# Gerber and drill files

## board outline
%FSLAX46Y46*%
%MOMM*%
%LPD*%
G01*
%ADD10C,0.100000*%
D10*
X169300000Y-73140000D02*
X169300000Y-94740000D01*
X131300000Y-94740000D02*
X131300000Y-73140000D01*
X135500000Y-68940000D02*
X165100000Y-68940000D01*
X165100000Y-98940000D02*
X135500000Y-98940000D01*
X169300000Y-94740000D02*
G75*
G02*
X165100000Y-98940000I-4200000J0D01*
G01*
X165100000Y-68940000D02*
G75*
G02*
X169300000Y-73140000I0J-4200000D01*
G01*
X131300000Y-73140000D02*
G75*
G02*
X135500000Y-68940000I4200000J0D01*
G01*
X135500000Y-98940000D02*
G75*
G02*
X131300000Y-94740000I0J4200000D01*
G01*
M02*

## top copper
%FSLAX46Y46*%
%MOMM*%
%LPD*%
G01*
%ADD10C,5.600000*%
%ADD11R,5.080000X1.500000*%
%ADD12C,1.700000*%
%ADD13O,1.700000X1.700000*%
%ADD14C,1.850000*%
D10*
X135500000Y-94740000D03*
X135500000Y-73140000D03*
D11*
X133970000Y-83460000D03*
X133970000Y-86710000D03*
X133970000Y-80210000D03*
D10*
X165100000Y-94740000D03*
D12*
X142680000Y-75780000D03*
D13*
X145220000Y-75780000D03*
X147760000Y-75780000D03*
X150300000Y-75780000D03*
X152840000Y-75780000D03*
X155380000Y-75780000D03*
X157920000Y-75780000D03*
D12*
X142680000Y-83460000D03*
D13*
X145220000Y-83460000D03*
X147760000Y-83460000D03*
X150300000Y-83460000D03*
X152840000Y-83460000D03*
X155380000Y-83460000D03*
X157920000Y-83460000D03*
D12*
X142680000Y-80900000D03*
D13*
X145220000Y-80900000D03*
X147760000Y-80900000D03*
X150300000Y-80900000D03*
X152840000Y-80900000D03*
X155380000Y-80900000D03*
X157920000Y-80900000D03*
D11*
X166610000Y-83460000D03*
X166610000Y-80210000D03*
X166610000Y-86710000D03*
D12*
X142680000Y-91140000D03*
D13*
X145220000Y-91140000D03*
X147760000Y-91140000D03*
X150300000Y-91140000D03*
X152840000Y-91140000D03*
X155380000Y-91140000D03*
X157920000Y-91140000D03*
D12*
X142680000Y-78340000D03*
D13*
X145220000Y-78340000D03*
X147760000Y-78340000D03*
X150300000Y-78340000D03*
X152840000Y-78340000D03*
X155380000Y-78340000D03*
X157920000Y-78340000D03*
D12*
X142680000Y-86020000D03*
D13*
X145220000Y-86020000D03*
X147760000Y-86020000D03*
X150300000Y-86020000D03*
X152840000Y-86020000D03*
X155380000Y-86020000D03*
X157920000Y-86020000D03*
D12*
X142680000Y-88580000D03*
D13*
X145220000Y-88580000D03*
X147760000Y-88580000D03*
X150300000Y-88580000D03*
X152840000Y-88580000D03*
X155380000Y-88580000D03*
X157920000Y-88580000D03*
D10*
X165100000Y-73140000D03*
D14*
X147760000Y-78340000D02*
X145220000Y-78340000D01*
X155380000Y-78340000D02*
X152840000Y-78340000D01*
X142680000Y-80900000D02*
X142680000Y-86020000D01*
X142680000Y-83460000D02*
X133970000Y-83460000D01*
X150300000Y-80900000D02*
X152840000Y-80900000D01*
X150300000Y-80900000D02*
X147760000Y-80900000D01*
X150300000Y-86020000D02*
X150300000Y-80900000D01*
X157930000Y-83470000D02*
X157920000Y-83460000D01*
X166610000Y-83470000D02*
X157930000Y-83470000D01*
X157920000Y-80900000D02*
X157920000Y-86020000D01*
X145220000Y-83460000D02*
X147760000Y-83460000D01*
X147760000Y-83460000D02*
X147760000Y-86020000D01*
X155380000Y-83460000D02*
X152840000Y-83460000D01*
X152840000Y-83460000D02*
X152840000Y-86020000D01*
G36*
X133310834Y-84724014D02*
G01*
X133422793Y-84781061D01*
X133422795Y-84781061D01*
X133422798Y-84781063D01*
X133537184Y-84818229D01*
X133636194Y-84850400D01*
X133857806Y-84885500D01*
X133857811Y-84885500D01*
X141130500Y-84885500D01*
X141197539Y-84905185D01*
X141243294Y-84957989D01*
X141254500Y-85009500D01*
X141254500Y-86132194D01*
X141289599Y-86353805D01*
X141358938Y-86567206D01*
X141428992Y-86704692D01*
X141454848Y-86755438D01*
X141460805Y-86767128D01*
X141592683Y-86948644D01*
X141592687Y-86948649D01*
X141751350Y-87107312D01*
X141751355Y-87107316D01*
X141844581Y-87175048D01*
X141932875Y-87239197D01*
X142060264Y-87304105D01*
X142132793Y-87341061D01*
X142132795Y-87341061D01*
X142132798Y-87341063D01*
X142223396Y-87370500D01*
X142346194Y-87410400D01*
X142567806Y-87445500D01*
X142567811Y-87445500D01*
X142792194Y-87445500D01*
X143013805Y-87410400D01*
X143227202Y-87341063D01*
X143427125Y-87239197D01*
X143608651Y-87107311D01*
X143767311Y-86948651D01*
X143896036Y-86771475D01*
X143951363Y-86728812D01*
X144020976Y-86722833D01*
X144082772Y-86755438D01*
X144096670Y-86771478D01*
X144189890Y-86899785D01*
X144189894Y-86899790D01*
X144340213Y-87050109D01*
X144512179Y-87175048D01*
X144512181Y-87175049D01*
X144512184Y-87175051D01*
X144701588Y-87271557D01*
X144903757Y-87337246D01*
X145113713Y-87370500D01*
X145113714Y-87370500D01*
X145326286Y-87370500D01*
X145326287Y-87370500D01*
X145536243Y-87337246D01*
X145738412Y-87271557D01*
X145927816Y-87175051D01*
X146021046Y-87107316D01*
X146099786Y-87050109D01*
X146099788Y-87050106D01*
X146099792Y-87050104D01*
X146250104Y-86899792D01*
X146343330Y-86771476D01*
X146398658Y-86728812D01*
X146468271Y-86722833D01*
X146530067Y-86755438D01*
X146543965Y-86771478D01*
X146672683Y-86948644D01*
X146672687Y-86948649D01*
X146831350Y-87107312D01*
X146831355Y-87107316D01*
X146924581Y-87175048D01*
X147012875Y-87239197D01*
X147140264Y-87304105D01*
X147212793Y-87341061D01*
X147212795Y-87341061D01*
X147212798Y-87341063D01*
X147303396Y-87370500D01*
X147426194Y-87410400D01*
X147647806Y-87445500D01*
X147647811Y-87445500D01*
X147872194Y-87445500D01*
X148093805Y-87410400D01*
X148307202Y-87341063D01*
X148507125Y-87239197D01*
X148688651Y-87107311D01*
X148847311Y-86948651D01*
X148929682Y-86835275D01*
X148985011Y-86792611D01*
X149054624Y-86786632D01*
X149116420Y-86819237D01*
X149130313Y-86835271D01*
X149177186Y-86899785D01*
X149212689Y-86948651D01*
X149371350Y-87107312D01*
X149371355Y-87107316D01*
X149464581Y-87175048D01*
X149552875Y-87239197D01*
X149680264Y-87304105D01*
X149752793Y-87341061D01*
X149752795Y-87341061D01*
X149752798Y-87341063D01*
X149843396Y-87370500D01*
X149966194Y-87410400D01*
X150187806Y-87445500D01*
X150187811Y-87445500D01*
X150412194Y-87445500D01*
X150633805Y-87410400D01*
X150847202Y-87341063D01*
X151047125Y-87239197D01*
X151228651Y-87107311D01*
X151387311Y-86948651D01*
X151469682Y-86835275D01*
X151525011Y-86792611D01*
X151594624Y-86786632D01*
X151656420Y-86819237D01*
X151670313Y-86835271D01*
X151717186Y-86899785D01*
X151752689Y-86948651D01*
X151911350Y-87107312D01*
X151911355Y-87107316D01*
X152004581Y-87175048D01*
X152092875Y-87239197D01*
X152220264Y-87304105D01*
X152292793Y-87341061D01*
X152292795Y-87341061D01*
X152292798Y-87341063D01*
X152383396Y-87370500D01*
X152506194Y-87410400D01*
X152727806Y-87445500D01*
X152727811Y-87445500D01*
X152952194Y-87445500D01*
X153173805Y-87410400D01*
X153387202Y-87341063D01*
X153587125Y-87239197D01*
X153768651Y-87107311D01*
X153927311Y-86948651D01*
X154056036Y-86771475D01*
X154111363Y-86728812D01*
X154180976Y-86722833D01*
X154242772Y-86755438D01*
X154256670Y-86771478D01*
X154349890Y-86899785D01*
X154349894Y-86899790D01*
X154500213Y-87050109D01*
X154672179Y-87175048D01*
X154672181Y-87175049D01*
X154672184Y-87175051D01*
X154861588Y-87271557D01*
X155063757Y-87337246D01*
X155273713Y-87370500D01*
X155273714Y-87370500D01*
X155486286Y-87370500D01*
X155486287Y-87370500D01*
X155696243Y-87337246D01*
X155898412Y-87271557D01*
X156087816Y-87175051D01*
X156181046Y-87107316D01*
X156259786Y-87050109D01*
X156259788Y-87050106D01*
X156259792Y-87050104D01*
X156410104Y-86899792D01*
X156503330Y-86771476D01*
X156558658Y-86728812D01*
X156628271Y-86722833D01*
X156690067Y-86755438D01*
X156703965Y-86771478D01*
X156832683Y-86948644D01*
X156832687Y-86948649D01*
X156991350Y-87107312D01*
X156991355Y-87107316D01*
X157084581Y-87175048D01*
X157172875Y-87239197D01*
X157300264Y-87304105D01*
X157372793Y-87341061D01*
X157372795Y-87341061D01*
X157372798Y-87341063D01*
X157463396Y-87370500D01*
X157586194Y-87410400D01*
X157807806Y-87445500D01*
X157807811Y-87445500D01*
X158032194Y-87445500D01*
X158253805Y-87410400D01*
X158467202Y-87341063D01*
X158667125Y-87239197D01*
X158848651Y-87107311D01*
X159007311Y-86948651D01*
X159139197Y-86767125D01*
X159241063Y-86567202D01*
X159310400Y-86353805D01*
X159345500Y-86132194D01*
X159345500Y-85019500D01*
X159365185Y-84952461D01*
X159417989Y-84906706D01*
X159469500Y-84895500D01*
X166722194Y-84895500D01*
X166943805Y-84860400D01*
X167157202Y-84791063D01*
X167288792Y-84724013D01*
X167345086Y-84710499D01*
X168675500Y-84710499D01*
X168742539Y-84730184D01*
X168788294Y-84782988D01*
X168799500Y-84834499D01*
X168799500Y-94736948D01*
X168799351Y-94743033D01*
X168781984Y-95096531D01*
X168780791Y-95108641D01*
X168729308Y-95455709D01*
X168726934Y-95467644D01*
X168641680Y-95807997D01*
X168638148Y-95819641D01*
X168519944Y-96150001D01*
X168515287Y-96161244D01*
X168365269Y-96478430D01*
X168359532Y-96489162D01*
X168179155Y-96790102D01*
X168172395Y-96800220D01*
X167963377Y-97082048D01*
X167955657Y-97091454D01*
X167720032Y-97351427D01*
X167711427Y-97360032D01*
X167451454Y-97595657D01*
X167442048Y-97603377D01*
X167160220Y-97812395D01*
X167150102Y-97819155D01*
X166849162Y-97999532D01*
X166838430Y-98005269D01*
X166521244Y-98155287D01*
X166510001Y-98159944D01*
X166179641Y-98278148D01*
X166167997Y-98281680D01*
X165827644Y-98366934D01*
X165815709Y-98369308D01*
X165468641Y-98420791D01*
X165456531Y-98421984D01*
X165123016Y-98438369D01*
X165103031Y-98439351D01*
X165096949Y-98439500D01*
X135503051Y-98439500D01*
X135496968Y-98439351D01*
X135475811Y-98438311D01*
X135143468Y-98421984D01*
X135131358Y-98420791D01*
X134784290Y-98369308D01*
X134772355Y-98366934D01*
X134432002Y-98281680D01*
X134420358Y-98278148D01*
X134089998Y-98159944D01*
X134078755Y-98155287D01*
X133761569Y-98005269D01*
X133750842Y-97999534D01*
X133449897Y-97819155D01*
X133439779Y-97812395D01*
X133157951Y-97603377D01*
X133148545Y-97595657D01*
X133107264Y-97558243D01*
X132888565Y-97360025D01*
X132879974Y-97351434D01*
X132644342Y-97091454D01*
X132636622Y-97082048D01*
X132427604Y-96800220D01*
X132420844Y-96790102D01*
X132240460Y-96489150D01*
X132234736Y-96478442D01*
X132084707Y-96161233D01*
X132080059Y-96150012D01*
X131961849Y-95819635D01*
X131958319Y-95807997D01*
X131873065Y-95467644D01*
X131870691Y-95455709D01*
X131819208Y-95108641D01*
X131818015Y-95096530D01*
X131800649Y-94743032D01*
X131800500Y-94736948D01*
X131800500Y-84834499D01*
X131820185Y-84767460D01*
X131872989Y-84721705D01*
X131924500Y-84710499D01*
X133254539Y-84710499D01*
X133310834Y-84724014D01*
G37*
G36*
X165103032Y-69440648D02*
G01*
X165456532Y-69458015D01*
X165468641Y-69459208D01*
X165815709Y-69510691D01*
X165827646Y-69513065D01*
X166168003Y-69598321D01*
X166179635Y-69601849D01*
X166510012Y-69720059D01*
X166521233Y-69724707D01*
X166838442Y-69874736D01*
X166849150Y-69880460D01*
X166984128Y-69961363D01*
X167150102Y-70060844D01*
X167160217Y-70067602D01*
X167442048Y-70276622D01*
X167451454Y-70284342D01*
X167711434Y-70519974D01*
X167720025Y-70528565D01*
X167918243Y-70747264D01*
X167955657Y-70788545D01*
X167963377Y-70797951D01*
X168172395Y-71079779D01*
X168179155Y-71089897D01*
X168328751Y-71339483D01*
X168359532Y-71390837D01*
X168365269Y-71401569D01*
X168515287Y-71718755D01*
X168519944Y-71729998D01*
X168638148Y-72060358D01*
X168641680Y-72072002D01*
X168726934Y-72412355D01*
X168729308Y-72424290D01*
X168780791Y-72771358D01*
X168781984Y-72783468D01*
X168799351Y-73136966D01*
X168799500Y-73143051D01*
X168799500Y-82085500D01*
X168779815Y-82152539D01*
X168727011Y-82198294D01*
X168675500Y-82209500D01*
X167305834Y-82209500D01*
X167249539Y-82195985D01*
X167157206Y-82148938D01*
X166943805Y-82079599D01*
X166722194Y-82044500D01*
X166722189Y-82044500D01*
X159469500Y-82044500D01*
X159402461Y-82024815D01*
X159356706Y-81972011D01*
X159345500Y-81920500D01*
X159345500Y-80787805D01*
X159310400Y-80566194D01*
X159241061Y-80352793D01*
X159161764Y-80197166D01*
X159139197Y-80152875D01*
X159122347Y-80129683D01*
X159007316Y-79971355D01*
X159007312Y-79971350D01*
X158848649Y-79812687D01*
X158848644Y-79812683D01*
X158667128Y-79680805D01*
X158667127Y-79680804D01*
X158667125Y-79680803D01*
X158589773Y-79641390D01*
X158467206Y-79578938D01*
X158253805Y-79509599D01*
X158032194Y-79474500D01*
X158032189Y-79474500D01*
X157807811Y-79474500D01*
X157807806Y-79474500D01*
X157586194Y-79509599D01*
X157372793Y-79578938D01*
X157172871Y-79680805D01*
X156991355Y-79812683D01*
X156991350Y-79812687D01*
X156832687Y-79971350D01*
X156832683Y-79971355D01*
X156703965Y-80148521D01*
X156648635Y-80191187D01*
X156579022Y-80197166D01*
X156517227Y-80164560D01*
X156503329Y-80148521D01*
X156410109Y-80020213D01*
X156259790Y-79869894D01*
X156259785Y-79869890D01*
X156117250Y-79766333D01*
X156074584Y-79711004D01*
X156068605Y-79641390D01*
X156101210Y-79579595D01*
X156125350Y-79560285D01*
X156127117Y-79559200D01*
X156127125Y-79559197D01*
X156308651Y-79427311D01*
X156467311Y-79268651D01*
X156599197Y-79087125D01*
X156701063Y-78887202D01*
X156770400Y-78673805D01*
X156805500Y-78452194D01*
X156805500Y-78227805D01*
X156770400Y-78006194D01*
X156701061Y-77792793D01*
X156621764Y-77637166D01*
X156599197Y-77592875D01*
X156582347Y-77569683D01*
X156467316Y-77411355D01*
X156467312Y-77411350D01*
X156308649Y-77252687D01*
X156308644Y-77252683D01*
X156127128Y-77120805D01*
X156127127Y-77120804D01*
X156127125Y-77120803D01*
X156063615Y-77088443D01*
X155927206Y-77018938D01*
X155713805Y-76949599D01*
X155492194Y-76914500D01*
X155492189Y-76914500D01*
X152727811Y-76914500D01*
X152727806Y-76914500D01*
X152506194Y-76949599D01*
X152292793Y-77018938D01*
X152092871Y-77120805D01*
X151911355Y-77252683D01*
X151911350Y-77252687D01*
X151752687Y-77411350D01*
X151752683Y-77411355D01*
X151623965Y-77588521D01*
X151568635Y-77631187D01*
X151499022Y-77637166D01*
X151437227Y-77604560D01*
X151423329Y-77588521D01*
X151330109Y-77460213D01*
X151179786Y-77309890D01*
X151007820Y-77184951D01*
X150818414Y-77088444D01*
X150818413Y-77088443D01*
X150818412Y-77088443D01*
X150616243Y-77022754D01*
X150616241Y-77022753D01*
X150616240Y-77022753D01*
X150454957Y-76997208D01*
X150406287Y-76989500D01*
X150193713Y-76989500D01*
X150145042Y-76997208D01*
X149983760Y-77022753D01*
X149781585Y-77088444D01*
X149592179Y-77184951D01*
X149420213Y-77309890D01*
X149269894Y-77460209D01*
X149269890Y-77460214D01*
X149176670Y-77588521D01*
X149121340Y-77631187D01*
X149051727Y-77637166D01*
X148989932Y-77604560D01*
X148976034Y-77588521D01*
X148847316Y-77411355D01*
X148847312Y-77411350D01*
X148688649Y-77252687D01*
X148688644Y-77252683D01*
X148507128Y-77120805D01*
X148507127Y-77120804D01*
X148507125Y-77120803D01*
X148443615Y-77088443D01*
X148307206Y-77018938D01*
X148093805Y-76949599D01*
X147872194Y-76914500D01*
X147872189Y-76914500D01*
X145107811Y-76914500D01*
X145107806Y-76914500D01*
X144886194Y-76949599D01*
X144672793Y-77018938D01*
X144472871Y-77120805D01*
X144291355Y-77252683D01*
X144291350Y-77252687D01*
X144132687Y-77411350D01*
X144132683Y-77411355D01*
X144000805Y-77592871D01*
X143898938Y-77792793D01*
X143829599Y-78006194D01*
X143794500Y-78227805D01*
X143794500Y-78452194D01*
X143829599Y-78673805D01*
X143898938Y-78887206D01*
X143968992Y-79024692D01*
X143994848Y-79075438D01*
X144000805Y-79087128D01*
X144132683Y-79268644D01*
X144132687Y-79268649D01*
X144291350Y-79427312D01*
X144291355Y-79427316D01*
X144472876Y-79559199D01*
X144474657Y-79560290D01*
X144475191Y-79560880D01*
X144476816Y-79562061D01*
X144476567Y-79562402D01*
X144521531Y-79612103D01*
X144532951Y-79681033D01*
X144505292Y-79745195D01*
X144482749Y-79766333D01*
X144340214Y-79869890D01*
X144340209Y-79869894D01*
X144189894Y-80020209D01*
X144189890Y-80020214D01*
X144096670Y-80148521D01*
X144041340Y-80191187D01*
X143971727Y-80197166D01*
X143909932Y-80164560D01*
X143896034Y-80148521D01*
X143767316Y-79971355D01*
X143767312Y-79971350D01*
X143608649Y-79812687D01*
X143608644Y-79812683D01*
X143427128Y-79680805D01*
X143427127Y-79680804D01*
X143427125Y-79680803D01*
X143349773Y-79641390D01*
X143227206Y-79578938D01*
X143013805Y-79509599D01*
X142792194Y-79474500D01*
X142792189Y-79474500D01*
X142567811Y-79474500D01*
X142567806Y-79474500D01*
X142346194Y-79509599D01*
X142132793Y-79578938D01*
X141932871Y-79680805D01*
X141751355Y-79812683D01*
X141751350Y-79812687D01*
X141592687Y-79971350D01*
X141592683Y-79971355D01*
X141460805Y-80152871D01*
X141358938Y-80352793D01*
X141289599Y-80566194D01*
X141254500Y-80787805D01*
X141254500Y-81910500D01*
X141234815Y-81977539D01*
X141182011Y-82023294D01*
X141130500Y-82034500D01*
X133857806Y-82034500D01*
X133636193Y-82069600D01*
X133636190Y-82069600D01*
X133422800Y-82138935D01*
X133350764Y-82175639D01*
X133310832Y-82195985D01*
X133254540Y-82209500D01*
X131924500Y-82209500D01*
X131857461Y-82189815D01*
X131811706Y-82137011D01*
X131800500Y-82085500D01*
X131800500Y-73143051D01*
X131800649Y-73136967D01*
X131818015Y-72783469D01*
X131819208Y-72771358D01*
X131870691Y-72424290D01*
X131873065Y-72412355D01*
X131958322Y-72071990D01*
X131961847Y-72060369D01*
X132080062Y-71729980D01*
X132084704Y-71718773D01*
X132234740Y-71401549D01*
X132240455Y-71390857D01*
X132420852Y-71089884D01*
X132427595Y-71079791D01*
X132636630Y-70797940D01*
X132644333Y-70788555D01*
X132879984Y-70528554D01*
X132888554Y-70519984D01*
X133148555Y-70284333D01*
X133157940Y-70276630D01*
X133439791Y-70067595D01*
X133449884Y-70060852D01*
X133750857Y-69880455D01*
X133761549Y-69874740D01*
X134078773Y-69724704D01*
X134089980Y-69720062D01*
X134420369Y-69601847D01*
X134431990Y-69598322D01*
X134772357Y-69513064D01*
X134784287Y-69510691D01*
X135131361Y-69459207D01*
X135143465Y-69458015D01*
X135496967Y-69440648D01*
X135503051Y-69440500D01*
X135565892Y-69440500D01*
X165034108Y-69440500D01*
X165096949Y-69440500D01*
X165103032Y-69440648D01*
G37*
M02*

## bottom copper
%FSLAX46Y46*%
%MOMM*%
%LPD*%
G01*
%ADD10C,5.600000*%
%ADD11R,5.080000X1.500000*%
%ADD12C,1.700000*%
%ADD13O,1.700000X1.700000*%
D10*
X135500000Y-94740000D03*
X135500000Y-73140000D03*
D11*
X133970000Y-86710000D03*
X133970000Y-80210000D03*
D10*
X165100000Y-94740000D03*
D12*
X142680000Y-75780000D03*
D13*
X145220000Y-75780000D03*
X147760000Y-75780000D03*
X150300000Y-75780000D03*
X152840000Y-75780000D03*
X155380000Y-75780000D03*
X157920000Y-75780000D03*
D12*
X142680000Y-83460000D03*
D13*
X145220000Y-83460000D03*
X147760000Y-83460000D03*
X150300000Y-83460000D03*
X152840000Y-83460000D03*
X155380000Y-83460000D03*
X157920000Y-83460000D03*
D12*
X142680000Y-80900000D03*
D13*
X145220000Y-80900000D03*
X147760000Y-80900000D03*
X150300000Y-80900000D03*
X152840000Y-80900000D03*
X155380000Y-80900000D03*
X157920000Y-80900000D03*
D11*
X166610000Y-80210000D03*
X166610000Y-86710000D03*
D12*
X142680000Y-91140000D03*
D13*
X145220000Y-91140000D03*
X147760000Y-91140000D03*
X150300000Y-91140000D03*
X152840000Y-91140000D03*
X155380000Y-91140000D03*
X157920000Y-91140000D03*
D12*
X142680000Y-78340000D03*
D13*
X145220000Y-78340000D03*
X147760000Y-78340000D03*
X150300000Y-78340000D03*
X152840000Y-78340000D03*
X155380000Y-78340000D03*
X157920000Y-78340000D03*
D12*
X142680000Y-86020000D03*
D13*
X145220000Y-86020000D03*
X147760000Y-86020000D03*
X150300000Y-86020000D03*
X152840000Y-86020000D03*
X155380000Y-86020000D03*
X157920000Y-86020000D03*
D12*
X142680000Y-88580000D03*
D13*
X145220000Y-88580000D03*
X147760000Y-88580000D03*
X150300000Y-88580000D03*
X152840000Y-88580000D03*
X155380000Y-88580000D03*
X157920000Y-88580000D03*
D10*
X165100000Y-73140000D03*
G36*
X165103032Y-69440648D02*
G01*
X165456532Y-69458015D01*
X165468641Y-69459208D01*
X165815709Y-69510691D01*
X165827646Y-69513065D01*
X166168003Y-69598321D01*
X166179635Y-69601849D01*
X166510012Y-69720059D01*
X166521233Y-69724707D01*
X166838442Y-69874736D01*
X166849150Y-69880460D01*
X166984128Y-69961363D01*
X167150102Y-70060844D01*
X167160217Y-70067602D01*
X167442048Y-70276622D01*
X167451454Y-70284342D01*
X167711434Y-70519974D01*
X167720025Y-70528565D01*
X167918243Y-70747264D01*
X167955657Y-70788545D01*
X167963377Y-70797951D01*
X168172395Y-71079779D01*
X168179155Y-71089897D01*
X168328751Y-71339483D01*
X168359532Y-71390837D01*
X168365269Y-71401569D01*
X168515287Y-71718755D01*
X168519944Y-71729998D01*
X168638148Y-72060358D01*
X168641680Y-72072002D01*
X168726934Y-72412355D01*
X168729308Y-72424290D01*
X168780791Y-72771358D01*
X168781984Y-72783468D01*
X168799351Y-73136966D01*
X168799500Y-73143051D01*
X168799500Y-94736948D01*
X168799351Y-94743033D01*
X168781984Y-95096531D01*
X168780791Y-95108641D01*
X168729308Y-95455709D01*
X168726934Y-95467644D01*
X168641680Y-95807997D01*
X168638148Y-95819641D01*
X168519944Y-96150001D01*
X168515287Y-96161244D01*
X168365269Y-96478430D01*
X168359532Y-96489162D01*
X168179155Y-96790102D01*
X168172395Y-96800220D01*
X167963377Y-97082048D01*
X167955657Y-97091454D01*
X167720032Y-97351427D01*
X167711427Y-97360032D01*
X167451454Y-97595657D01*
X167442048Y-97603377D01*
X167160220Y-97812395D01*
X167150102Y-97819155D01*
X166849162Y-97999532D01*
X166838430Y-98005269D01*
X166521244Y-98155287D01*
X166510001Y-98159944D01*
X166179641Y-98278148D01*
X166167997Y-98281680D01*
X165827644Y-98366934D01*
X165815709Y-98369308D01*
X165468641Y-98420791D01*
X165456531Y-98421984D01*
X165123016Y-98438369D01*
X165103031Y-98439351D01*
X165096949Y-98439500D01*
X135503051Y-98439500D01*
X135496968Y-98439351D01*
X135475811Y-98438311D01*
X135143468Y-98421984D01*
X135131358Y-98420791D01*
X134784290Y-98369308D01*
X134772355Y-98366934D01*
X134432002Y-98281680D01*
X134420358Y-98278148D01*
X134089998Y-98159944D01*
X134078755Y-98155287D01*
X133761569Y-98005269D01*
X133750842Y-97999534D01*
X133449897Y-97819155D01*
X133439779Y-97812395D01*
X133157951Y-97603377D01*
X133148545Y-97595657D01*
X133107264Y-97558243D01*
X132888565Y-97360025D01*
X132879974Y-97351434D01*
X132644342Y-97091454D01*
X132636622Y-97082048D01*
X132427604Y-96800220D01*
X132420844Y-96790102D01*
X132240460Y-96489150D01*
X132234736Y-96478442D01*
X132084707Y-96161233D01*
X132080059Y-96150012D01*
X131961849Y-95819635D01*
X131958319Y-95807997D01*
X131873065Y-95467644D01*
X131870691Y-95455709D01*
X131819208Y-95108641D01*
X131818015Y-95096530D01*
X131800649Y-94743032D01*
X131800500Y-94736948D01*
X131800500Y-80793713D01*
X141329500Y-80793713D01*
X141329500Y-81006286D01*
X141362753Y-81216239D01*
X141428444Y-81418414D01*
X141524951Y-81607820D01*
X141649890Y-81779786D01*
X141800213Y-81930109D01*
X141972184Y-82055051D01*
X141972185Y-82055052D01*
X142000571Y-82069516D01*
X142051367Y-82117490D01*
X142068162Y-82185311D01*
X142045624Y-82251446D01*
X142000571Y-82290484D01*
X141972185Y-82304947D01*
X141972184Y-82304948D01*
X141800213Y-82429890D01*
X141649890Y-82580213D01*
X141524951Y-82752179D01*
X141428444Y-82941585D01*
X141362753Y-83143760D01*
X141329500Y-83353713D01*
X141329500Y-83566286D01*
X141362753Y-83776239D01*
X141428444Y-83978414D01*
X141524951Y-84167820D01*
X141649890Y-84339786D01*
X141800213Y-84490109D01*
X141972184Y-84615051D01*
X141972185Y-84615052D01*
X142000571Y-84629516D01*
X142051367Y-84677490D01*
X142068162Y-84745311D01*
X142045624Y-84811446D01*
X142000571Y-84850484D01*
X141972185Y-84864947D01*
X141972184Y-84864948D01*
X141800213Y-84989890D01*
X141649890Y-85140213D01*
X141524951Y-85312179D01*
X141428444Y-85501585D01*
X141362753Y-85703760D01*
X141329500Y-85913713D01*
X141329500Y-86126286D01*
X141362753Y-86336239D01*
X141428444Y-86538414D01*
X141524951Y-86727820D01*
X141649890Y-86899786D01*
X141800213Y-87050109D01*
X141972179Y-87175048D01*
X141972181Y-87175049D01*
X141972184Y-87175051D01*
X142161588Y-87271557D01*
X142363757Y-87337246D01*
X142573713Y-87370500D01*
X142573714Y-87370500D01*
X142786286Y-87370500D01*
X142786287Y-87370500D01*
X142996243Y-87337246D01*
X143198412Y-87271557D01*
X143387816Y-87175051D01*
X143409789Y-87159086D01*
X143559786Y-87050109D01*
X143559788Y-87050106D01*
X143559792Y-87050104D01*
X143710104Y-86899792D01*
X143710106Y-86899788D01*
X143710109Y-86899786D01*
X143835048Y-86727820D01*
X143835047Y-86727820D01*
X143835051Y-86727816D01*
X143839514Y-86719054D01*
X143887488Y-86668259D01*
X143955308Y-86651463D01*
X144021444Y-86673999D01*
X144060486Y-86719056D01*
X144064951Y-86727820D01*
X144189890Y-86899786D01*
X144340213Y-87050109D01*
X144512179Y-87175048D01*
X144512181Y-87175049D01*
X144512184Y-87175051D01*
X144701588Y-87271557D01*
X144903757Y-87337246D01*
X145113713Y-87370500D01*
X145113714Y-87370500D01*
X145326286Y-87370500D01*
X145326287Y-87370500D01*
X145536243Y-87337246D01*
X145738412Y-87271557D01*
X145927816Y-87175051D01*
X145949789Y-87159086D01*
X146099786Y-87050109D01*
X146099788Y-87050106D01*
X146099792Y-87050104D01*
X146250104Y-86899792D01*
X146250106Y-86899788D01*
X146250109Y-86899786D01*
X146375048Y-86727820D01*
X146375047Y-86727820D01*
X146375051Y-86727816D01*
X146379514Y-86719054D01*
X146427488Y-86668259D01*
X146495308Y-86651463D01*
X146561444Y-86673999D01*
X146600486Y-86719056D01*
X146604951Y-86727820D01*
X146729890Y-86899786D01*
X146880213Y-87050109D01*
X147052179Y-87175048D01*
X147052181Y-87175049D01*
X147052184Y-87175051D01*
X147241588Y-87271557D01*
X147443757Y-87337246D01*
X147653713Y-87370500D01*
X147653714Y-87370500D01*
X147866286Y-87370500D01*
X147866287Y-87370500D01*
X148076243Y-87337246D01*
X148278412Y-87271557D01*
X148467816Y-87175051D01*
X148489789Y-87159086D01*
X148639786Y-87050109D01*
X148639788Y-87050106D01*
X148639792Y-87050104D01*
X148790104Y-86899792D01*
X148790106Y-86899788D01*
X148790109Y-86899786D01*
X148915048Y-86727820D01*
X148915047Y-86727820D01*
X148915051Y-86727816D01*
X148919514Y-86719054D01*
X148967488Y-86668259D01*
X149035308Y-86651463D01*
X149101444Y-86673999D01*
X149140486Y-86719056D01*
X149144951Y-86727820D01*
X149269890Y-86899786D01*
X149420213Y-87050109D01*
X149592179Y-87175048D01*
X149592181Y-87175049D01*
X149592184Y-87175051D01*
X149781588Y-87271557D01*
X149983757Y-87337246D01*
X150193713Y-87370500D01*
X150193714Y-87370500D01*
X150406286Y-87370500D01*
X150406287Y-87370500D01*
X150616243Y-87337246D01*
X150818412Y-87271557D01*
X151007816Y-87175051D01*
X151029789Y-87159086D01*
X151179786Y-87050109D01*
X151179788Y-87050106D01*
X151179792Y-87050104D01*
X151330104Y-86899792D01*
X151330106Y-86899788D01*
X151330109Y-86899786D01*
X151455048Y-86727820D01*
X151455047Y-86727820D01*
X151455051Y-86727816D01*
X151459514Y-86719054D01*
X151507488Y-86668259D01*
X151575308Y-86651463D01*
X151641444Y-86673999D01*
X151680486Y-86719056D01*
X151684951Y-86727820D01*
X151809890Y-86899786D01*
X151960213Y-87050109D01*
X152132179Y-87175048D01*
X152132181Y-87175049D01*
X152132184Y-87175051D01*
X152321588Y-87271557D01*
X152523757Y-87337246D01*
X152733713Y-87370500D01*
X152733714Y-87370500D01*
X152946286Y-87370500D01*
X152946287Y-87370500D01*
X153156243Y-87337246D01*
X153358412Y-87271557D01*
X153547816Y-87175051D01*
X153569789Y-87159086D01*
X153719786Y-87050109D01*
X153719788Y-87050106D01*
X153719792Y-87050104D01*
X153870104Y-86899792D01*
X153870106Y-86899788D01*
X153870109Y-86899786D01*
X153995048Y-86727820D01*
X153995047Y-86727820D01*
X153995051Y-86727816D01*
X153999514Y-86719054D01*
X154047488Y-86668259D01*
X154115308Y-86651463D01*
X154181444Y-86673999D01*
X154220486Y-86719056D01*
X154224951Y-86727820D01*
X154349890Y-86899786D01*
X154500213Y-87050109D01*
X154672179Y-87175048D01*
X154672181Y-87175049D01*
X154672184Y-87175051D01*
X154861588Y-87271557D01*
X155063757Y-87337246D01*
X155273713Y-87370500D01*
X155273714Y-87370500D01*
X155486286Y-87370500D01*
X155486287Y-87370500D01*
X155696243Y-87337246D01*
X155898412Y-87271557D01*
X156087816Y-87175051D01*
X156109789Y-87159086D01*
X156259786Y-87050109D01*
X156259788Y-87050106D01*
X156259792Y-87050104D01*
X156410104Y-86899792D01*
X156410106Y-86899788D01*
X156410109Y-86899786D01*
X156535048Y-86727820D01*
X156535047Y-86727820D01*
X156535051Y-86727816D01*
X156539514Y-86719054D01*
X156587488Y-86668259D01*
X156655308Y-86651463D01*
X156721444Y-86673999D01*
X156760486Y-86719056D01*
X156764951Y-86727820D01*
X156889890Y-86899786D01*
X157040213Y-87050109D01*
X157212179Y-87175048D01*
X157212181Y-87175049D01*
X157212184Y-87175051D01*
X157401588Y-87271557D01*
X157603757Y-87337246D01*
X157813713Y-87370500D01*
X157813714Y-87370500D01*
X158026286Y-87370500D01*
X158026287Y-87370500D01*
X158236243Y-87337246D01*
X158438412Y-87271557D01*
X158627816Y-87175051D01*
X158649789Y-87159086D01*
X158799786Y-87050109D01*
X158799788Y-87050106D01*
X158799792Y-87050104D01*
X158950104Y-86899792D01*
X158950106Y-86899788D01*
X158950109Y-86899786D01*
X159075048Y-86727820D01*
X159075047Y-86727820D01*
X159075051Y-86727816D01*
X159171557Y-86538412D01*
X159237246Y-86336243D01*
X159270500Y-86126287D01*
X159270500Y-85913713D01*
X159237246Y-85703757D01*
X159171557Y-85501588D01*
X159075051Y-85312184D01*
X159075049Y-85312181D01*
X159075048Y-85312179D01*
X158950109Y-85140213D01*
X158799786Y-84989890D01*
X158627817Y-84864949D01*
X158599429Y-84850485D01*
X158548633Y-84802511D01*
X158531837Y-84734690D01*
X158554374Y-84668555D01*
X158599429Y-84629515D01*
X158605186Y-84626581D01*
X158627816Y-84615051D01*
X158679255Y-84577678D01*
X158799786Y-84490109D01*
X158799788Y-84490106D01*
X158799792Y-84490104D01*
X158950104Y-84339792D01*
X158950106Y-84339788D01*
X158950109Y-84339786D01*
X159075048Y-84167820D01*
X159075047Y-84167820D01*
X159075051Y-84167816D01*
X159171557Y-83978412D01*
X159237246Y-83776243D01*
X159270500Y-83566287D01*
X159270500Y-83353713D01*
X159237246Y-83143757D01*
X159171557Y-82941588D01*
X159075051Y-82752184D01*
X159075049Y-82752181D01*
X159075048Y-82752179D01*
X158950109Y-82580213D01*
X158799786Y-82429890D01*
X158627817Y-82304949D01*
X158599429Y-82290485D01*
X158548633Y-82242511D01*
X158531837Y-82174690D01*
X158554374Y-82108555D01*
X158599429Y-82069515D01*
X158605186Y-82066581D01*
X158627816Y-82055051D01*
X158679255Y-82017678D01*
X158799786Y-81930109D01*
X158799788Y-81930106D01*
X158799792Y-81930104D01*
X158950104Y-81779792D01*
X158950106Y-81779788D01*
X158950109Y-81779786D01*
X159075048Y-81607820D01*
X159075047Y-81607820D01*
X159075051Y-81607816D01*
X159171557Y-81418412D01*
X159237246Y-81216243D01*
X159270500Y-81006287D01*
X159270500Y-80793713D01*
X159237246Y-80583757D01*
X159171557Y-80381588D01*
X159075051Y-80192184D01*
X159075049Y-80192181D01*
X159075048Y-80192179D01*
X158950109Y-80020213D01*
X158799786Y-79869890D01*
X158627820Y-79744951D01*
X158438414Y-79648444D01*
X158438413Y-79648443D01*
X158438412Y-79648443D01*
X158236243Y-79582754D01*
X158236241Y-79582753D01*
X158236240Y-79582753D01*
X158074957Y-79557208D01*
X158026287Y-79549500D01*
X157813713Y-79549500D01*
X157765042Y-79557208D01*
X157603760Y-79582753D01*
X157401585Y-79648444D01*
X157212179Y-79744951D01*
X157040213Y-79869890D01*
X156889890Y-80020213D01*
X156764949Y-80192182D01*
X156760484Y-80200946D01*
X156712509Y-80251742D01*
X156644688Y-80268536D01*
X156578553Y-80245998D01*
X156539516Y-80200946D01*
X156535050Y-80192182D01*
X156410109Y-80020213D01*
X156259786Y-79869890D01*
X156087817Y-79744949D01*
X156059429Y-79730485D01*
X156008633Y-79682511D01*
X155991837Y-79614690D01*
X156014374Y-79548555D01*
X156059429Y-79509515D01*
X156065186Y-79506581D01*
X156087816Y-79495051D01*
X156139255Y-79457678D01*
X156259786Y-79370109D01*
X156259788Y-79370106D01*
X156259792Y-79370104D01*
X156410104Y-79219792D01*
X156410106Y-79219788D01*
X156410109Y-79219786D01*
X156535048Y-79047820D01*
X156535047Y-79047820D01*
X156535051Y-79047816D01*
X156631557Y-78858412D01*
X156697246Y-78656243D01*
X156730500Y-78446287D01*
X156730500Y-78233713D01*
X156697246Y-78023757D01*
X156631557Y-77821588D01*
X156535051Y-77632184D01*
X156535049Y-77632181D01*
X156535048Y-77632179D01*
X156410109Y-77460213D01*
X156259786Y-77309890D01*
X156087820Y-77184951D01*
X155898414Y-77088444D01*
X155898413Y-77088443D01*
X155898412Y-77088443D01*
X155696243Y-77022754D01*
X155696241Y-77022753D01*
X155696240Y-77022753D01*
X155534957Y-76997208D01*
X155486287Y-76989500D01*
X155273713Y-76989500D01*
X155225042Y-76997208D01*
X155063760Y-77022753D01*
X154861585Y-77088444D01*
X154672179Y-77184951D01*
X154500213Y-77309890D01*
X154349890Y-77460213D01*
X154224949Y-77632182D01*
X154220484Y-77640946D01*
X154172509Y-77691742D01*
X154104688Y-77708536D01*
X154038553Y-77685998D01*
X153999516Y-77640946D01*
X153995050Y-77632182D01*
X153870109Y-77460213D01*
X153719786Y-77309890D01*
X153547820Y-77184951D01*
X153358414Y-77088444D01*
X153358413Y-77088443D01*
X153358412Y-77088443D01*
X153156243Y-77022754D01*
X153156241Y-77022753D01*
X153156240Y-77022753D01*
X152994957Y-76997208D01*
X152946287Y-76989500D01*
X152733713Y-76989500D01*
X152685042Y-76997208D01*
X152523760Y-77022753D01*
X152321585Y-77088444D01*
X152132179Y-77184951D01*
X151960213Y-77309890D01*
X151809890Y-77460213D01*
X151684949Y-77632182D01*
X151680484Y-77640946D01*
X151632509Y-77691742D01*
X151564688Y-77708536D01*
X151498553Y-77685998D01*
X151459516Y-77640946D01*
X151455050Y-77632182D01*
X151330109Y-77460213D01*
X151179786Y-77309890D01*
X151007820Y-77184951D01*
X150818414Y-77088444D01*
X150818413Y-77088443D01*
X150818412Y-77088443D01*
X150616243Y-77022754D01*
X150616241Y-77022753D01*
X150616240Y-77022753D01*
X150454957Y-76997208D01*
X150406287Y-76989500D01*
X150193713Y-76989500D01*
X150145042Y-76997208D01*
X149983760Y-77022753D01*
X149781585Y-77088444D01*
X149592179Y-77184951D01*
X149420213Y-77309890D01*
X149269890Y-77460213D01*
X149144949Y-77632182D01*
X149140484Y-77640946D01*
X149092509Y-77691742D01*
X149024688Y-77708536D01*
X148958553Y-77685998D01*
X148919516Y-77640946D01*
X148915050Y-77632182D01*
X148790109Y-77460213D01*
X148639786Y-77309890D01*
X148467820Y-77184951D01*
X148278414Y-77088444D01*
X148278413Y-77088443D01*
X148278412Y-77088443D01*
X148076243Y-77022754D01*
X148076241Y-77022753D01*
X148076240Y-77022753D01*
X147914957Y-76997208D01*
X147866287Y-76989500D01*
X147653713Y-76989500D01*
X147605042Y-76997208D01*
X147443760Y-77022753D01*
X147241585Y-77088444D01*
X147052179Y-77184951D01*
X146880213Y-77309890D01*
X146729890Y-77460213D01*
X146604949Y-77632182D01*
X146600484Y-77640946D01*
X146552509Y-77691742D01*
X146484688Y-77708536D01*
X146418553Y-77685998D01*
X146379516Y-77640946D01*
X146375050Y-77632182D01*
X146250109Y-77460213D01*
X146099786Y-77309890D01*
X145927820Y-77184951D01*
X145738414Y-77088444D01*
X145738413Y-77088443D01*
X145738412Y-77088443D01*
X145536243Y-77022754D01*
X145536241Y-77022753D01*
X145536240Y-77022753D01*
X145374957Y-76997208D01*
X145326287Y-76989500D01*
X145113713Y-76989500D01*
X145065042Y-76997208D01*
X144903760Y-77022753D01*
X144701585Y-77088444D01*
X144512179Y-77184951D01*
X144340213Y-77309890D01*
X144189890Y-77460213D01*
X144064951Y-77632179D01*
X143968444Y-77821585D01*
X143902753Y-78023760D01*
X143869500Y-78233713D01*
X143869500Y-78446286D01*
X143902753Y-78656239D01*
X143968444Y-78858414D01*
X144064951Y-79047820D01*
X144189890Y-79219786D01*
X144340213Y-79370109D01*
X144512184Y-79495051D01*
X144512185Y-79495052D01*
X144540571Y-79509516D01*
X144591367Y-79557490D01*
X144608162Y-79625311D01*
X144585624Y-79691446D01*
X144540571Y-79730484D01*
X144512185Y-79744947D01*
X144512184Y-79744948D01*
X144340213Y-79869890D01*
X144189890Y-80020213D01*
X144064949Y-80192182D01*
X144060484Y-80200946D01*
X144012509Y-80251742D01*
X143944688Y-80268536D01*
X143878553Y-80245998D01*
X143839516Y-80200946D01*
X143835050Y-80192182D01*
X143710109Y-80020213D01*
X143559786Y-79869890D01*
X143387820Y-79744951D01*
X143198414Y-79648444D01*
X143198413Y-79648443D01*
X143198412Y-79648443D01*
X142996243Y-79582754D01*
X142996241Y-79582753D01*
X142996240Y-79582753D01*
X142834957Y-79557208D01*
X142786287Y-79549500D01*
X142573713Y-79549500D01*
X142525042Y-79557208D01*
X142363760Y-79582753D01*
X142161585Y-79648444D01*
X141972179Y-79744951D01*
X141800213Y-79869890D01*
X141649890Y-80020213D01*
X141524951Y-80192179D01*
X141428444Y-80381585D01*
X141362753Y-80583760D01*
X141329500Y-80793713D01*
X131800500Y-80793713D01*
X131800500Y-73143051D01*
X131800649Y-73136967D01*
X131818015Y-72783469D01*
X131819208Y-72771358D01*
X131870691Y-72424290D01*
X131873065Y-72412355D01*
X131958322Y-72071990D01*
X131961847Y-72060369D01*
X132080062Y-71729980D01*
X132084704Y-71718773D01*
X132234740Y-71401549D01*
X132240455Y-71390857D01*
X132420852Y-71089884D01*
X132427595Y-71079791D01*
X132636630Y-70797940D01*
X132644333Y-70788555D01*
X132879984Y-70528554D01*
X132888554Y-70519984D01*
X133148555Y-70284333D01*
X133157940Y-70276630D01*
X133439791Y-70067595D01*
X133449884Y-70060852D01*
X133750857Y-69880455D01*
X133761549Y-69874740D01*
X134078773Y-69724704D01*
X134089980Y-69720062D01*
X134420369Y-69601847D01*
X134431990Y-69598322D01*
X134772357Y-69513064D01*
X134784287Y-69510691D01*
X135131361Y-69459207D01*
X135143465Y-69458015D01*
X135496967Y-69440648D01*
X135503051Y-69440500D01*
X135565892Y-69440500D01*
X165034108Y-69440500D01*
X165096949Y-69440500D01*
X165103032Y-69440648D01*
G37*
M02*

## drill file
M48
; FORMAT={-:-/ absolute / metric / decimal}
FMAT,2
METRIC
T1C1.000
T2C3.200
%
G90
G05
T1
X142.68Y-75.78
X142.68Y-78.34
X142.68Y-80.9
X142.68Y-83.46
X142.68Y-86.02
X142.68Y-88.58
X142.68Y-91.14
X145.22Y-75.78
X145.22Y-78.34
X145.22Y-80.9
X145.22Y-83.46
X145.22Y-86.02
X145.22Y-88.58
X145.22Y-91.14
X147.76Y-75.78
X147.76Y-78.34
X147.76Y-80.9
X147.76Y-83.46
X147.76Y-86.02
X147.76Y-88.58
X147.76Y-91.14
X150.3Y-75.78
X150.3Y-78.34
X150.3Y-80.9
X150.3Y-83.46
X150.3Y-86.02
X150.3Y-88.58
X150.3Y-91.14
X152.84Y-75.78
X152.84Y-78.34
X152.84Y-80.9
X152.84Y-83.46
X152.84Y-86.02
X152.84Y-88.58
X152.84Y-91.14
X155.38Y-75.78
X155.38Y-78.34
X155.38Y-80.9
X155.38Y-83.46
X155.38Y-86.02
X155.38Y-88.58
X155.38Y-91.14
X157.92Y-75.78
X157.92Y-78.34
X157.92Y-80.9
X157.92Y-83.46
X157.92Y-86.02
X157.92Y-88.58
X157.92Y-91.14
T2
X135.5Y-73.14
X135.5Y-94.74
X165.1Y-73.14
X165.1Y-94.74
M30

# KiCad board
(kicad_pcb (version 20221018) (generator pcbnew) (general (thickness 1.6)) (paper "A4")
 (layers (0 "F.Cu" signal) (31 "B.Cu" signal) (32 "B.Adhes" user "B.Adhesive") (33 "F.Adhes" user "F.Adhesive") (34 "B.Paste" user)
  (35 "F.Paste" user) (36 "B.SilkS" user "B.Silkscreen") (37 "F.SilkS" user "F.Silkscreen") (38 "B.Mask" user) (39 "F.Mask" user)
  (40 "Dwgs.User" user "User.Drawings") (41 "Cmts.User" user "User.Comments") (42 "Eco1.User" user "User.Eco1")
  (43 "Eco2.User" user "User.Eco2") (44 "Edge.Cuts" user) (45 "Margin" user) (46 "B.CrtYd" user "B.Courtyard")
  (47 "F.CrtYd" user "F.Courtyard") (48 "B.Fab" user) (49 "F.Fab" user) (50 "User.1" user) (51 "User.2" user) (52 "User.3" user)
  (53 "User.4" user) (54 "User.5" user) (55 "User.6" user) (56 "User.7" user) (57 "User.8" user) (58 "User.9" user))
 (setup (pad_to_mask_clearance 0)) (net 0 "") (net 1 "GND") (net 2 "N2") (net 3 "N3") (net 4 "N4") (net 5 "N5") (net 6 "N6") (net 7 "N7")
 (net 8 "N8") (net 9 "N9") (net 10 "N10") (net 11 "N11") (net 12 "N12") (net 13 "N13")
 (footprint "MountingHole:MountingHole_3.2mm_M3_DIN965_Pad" (layer "F.Cu") (at 135.5 94.74)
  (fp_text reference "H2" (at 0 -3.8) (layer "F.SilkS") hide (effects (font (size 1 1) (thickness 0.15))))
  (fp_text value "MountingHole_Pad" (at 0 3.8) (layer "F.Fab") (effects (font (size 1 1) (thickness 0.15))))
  (pad "1" thru_hole circle (at 0 0) (size 5.6 5.6) (drill 3.2) (layers "*.Cu" "*.Mask") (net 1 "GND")))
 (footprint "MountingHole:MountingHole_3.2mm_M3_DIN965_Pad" (layer "F.Cu") (at 135.5 73.14)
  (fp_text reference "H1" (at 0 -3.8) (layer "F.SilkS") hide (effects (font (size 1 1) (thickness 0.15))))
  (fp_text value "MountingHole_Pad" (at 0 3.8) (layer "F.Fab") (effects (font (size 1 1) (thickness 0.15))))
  (pad "1" thru_hole circle (at 0 0) (size 5.6 5.6) (drill 3.2) (layers "*.Cu" "*.Mask") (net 1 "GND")))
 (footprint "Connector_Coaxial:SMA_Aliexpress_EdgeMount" (layer "F.Cu") (at 133.97 83.46 180)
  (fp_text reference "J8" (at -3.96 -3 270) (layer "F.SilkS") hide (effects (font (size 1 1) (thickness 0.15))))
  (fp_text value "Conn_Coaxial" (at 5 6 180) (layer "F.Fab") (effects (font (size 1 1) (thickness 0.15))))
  (pad "1" smd rect (at 0 0 270) (size 1.5 5.08) (layers "F.Cu" "F.Paste" "F.Mask") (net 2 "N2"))
  (pad "2" smd rect (at 0 -3.25 270) (size 1.5 5.08) (layers "F.Cu" "F.Paste" "F.Mask") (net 1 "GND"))
  (pad "2" smd rect (at 0 -3.25 270) (size 1.5 5.08) (layers "B.Cu" "B.Paste" "B.Mask") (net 1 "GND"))
  (pad "2" smd rect (at 0 3.25 270) (size 1.5 5.08) (layers "F.Cu" "F.Paste" "F.Mask") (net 1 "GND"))
  (pad "2" smd rect (at 0 3.25 270) (size 1.5 5.08) (layers "B.Cu" "B.Paste" "B.Mask") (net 1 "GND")))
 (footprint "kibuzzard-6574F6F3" (layer "F.Cu") (at 165.9 90.14)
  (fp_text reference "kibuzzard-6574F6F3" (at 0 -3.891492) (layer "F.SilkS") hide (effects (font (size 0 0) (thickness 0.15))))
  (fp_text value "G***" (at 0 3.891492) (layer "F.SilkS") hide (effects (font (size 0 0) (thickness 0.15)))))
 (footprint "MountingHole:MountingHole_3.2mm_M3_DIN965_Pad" (layer "F.Cu") (at 165.1 94.74)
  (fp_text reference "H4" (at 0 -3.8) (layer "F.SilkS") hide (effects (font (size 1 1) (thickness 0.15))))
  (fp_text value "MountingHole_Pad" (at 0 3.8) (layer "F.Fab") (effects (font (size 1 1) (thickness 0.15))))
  (pad "1" thru_hole circle (at 0 0) (size 5.6 5.6) (drill 3.2) (layers "*.Cu" "*.Mask") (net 1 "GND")))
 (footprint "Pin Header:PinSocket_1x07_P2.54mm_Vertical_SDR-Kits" (layer "F.Cu") (at 142.68 75.78 90)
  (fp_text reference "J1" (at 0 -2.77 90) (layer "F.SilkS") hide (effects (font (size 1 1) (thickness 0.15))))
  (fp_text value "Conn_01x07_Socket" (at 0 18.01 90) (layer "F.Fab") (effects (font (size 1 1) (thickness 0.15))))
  (pad "1" thru_hole circle (at 0 0 90) (size 1.7 1.7) (drill 1) (layers "*.Cu" "*.Mask") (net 1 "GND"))
  (pad "2" thru_hole oval (at 0 2.54 90) (size 1.7 1.7) (drill 1) (layers "*.Cu" "*.Mask") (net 1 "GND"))
  (pad "3" thru_hole oval (at 0 5.08 90) (size 1.7 1.7) (drill 1) (layers "*.Cu" "*.Mask") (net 1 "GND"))
  (pad "4" thru_hole oval (at 0 7.62 90) (size 1.7 1.7) (drill 1) (layers "*.Cu" "*.Mask") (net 1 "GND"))
  (pad "5" thru_hole oval (at 0 10.16 90) (size 1.7 1.7) (drill 1) (layers "*.Cu" "*.Mask") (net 1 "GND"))
  (pad "6" thru_hole oval (at 0 12.7 90) (size 1.7 1.7) (drill 1) (layers "*.Cu" "*.Mask") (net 1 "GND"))
  (pad "7" thru_hole oval (at 0 15.24 90) (size 1.7 1.7) (drill 1) (layers "*.Cu" "*.Mask") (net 1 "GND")))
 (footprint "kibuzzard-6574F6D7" (layer "F.Cu") (at 134.8 90.14)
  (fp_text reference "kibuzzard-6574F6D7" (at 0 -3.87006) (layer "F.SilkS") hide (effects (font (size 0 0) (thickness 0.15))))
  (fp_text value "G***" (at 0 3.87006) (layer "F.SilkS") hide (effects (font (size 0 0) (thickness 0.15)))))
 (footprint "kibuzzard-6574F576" (layer "F.Cu") (at 150.4 94.44)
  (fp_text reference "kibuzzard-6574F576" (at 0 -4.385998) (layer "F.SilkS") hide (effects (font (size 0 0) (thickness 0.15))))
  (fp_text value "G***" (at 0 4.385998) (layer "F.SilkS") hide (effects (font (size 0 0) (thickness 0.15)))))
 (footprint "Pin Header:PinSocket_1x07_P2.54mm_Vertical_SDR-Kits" (layer "F.Cu") (at 142.68 83.46 90)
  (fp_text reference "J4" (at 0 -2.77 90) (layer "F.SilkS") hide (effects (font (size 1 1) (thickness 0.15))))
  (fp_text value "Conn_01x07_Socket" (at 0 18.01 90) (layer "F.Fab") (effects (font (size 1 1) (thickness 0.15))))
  (pad "1" thru_hole circle (at 0 0 90) (size 1.7 1.7) (drill 1) (layers "*.Cu" "*.Mask") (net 2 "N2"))
  (pad "2" thru_hole oval (at 0 2.54 90) (size 1.7 1.7) (drill 1) (layers "*.Cu" "*.Mask") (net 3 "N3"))
  (pad "3" thru_hole oval (at 0 5.08 90) (size 1.7 1.7) (drill 1) (layers "*.Cu" "*.Mask") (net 3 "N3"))
  (pad "4" thru_hole oval (at 0 7.62 90) (size 1.7 1.7) (drill 1) (layers "*.Cu" "*.Mask") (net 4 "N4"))
  (pad "5" thru_hole oval (at 0 10.16 90) (size 1.7 1.7) (drill 1) (layers "*.Cu" "*.Mask") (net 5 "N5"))
  (pad "6" thru_hole oval (at 0 12.7 90) (size 1.7 1.7) (drill 1) (layers "*.Cu" "*.Mask") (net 5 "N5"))
  (pad "7" thru_hole oval (at 0 15.24 90) (size 1.7 1.7) (drill 1) (layers "*.Cu" "*.Mask") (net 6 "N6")))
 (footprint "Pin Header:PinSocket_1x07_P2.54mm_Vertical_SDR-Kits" (layer "F.Cu") (at 142.68 80.9 90)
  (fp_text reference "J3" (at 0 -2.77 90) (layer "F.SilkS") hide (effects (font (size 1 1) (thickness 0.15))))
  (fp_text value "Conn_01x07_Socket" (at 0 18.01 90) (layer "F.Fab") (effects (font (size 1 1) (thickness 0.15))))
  (pad "1" thru_hole circle (at 0 0 90) (size 1.7 1.7) (drill 1) (layers "*.Cu" "*.Mask") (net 2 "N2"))
  (pad "2" thru_hole oval (at 0 2.54 90) (size 1.7 1.7) (drill 1) (layers "*.Cu" "*.Mask") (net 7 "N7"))
  (pad "3" thru_hole oval (at 0 5.08 90) (size 1.7 1.7) (drill 1) (layers "*.Cu" "*.Mask") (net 4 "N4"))
  (pad "4" thru_hole oval (at 0 7.62 90) (size 1.7 1.7) (drill 1) (layers "*.Cu" "*.Mask") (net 4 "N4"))
  (pad "5" thru_hole oval (at 0 10.16 90) (size 1.7 1.7) (drill 1) (layers "*.Cu" "*.Mask") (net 4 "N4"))
  (pad "6" thru_hole oval (at 0 12.7 90) (size 1.7 1.7) (drill 1) (layers "*.Cu" "*.Mask") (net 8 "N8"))
  (pad "7" thru_hole oval (at 0 15.24 90) (size 1.7 1.7) (drill 1) (layers "*.Cu" "*.Mask") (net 6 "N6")))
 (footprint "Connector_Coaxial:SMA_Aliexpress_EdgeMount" (layer "F.Cu") (at 166.61 83.46)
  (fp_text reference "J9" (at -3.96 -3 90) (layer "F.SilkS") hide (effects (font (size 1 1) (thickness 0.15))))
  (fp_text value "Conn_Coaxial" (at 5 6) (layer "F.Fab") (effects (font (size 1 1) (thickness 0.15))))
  (pad "1" smd rect (at 0 0 90) (size 1.5 5.08) (layers "F.Cu" "F.Paste" "F.Mask") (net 6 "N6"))
  (pad "2" smd rect (at 0 -3.25 90) (size 1.5 5.08) (layers "F.Cu" "F.Paste" "F.Mask") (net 1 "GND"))
  (pad "2" smd rect (at 0 -3.25 90) (size 1.5 5.08) (layers "B.Cu" "B.Paste" "B.Mask") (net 1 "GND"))
  (pad "2" smd rect (at 0 3.25 90) (size 1.5 5.08) (layers "F.Cu" "F.Paste" "F.Mask") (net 1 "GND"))
  (pad "2" smd rect (at 0 3.25 90) (size 1.5 5.08) (layers "B.Cu" "B.Paste" "B.Mask") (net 1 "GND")))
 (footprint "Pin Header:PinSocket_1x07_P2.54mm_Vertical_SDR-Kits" (layer "F.Cu") (at 142.68 91.14 90)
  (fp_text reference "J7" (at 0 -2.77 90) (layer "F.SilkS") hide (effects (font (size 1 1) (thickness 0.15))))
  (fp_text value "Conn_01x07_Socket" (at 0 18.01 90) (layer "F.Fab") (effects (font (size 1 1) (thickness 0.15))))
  (pad "1" thru_hole circle (at 0 0 90) (size 1.7 1.7) (drill 1) (layers "*.Cu" "*.Mask") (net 1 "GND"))
  (pad "2" thru_hole oval (at 0 2.54 90) (size 1.7 1.7) (drill 1) (layers "*.Cu" "*.Mask") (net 1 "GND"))
  (pad "3" thru_hole oval (at 0 5.08 90) (size 1.7 1.7) (drill 1) (layers "*.Cu" "*.Mask") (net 1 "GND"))
  (pad "4" thru_hole oval (at 0 7.62 90) (size 1.7 1.7) (drill 1) (layers "*.Cu" "*.Mask") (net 1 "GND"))
  (pad "5" thru_hole oval (at 0 10.16 90) (size 1.7 1.7) (drill 1) (layers "*.Cu" "*.Mask") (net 1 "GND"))
  (pad "6" thru_hole oval (at 0 12.7 90) (size 1.7 1.7) (drill 1) (layers "*.Cu" "*.Mask") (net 1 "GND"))
  (pad "7" thru_hole oval (at 0 15.24 90) (size 1.7 1.7) (drill 1) (layers "*.Cu" "*.Mask") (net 1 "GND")))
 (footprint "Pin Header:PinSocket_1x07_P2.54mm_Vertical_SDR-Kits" (layer "F.Cu") (at 142.68 78.34 90)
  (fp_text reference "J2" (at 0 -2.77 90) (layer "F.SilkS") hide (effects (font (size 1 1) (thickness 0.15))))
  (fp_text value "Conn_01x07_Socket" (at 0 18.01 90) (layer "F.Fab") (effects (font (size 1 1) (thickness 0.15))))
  (pad "1" thru_hole circle (at 0 0 90) (size 1.7 1.7) (drill 1) (layers "*.Cu" "*.Mask") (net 1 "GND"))
  (pad "2" thru_hole oval (at 0 2.54 90) (size 1.7 1.7) (drill 1) (layers "*.Cu" "*.Mask") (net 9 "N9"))
  (pad "3" thru_hole oval (at 0 5.08 90) (size 1.7 1.7) (drill 1) (layers "*.Cu" "*.Mask") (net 9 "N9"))
  (pad "4" thru_hole oval (at 0 7.62 90) (size 1.7 1.7) (drill 1) (layers "*.Cu" "*.Mask") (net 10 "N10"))
  (pad "5" thru_hole oval (at 0 10.16 90) (size 1.7 1.7) (drill 1) (layers "*.Cu" "*.Mask") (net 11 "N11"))
  (pad "6" thru_hole oval (at 0 12.7 90) (size 1.7 1.7) (drill 1) (layers "*.Cu" "*.Mask") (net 11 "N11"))
  (pad "7" thru_hole oval (at 0 15.24 90) (size 1.7 1.7) (drill 1) (layers "*.Cu" "*.Mask") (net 1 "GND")))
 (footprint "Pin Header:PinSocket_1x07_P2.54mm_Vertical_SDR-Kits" (layer "F.Cu") (at 142.68 86.02 90)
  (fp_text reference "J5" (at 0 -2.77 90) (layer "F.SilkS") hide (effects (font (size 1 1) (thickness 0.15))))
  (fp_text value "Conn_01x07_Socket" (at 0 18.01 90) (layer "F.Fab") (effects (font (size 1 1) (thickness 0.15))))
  (pad "1" thru_hole circle (at 0 0 90) (size 1.7 1.7) (drill 1) (layers "*.Cu" "*.Mask") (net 2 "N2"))
  (pad "2" thru_hole oval (at 0 2.54 90) (size 1.7 1.7) (drill 1) (layers "*.Cu" "*.Mask") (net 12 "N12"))
  (pad "3" thru_hole oval (at 0 5.08 90) (size 1.7 1.7) (drill 1) (layers "*.Cu" "*.Mask") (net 3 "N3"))
  (pad "4" thru_hole oval (at 0 7.62 90) (size 1.7 1.7) (drill 1) (layers "*.Cu" "*.Mask") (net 4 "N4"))
  (pad "5" thru_hole oval (at 0 10.16 90) (size 1.7 1.7) (drill 1) (layers "*.Cu" "*.Mask") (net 5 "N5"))
  (pad "6" thru_hole oval (at 0 12.7 90) (size 1.7 1.7) (drill 1) (layers "*.Cu" "*.Mask") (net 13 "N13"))
  (pad "7" thru_hole oval (at 0 15.24 90) (size 1.7 1.7) (drill 1) (layers "*.Cu" "*.Mask") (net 6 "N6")))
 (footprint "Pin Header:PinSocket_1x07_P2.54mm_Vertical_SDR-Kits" (layer "F.Cu") (at 142.68 88.58 90)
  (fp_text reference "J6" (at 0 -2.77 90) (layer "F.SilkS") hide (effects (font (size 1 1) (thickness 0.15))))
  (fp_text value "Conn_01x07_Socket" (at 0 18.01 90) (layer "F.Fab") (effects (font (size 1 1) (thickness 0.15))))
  (pad "1" thru_hole circle (at 0 0 90) (size 1.7 1.7) (drill 1) (layers "*.Cu" "*.Mask") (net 1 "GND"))
  (pad "2" thru_hole oval (at 0 2.54 90) (size 1.7 1.7) (drill 1) (layers "*.Cu" "*.Mask") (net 1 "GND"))
  (pad "3" thru_hole oval (at 0 5.08 90) (size 1.7 1.7) (drill 1) (layers "*.Cu" "*.Mask") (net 1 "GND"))
  (pad "4" thru_hole oval (at 0 7.62 90) (size 1.7 1.7) (drill 1) (layers "*.Cu" "*.Mask") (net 1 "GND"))
  (pad "5" thru_hole oval (at 0 10.16 90) (size 1.7 1.7) (drill 1) (layers "*.Cu" "*.Mask") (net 1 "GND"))
  (pad "6" thru_hole oval (at 0 12.7 90) (size 1.7 1.7) (drill 1) (layers "*.Cu" "*.Mask") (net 1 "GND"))
  (pad "7" thru_hole oval (at 0 15.24 90) (size 1.7 1.7) (drill 1) (layers "*.Cu" "*.Mask") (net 1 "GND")))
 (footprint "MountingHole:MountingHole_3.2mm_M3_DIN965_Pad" (layer "F.Cu") (at 165.1 73.14)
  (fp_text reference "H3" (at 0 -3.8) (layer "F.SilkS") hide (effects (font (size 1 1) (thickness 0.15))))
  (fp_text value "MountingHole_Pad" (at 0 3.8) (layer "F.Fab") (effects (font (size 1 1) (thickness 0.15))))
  (pad "1" thru_hole circle (at 0 0) (size 5.6 5.6) (drill 3.2) (layers "*.Cu" "*.Mask") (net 1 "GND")))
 (gr_line (start 169.3 73.14) (end 169.3 94.74) (stroke (width 0.1) (type default)) (layer "Edge.Cuts"))
 (gr_line (start 131.3 94.74) (end 131.3 73.14) (stroke (width 0.1) (type default)) (layer "Edge.Cuts"))
 (gr_line (start 135.5 68.94) (end 165.1 68.94) (stroke (width 0.1) (type default)) (layer "Edge.Cuts"))
 (gr_line (start 165.1 98.94) (end 135.5 98.94) (stroke (width 0.1) (type default)) (layer "Edge.Cuts"))
 (gr_arc (start 169.3 94.74) (mid 168.069848 97.709848) (end 165.1 98.94) (stroke (width 0.1) (type default)) (layer "Edge.Cuts"))
 (gr_arc (start 165.1 68.94) (mid 168.069848 70.170152) (end 169.3 73.14) (stroke (width 0.1) (type default)) (layer "Edge.Cuts"))
 (gr_arc (start 131.3 73.14) (mid 132.530152 70.170152) (end 135.5 68.94) (stroke (width 0.1) (type default)) (layer "Edge.Cuts"))
 (gr_arc (start 135.5 98.94) (mid 132.530152 97.709848) (end 131.3 94.74) (stroke (width 0.1) (type default)) (layer "Edge.Cuts"))
 (segment (start 147.76 78.34) (end 145.22 78.34) (width 1.85) (layer "F.Cu") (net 9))
 (segment (start 155.38 78.34) (end 152.84 78.34) (width 1.85) (layer "F.Cu") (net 11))
 (segment (start 142.68 80.9) (end 142.68 86.02) (width 1.85) (layer "F.Cu") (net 2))
 (segment (start 142.68 83.46) (end 133.97 83.46) (width 1.85) (layer "F.Cu") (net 2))
 (segment (start 150.3 80.9) (end 152.84 80.9) (width 1.85) (layer "F.Cu") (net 4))
 (segment (start 150.3 80.9) (end 147.76 80.9) (width 1.85) (layer "F.Cu") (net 4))
 (segment (start 150.3 86.02) (end 150.3 80.9) (width 1.85) (layer "F.Cu") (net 4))
 (segment (start 157.93 83.47) (end 157.92 83.46) (width 1.85) (layer "F.Cu") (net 6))
 (segment (start 166.61 83.47) (end 157.93 83.47) (width 1.85) (layer "F.Cu") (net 6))
 (segment (start 157.92 80.9) (end 157.92 86.02) (width 1.85) (layer "F.Cu") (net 6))
 (segment (start 145.22 83.46) (end 147.76 83.46) (width 1.85) (layer "F.Cu") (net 3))
 (segment (start 147.76 83.46) (end 147.76 86.02) (width 1.85) (layer "F.Cu") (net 3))
 (segment (start 155.38 83.46) (end 152.84 83.46) (width 1.85) (layer "F.Cu") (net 5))
 (segment (start 152.84 83.46) (end 152.84 86.02) (width 1.85) (layer "F.Cu") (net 5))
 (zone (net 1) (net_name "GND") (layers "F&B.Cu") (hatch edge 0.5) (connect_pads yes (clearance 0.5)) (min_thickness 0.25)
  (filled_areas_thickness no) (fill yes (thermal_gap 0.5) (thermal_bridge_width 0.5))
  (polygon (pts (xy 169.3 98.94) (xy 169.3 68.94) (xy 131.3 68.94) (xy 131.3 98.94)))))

